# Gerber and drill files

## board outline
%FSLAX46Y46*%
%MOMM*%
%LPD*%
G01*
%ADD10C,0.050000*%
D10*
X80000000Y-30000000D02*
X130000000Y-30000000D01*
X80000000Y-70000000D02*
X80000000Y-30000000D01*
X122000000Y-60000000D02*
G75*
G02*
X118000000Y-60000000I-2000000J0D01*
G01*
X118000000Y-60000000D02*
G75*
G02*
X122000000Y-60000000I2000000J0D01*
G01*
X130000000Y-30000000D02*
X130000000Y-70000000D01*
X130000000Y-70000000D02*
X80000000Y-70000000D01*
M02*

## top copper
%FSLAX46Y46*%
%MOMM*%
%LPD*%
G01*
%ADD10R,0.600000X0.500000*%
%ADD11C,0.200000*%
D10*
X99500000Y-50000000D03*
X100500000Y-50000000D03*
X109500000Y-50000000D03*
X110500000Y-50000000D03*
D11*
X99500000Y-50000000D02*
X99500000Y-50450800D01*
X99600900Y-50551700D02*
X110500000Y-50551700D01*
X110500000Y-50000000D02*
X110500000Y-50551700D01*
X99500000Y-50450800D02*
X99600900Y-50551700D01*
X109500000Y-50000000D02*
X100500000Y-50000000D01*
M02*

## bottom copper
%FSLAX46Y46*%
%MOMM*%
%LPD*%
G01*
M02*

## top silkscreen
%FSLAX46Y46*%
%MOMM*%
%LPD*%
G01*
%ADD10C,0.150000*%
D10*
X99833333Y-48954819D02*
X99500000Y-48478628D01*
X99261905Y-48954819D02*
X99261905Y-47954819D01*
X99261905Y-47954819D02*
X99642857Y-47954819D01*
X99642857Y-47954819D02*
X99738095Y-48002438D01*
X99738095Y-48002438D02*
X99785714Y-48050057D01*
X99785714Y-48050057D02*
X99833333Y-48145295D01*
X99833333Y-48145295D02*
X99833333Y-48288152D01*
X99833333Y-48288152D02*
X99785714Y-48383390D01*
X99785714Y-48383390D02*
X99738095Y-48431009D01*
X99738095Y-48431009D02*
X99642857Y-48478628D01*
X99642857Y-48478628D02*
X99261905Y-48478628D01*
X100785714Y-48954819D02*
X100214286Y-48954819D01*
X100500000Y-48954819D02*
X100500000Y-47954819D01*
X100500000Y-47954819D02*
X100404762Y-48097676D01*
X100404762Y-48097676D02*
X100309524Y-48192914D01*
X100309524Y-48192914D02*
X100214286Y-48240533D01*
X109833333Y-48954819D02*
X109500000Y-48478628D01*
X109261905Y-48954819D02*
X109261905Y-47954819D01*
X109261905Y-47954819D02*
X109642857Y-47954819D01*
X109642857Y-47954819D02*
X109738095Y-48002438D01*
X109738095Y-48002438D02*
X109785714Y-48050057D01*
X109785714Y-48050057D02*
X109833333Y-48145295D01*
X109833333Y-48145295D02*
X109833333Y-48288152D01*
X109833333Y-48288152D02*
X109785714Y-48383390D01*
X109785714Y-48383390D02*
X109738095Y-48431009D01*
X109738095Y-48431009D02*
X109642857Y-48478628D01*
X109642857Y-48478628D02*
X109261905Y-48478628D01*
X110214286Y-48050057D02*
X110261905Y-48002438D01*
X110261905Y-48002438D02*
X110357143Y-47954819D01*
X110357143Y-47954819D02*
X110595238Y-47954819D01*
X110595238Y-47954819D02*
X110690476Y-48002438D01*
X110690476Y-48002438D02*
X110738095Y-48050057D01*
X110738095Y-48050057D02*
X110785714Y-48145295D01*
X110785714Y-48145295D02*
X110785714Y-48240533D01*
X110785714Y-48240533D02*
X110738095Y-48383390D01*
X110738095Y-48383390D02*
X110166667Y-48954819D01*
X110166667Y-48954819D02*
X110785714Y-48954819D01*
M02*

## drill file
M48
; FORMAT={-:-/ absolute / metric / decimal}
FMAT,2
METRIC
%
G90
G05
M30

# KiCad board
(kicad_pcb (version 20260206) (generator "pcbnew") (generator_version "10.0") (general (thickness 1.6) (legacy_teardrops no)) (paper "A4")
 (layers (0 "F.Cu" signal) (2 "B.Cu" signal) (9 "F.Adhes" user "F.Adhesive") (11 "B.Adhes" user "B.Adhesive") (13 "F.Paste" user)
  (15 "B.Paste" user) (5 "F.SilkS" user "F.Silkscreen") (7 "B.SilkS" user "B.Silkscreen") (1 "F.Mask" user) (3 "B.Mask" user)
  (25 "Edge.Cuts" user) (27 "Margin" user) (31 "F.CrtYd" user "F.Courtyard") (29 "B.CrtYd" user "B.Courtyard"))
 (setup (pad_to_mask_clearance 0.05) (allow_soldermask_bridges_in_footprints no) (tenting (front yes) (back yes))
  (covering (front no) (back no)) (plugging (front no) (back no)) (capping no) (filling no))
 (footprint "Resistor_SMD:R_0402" (layer "F.Cu") (at 100 50)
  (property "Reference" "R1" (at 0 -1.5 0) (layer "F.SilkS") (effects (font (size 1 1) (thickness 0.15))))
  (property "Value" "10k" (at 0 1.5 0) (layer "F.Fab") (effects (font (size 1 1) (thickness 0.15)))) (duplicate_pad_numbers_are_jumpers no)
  (pad "1" smd rect (at -0.5 0) (size 0.6 0.5) (layers "F.Cu" "F.Mask" "F.Paste") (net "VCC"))
  (pad "2" smd rect (at 0.5 0) (size 0.6 0.5) (layers "F.Cu" "F.Mask" "F.Paste") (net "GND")))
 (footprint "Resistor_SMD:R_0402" (layer "F.Cu") (at 110 50)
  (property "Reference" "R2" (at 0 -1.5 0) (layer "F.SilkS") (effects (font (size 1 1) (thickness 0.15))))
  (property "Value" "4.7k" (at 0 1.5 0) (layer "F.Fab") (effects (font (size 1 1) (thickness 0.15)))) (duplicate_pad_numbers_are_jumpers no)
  (pad "1" smd rect (at -0.5 0) (size 0.6 0.5) (layers "F.Cu" "F.Mask" "F.Paste") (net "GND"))
  (pad "2" smd rect (at 0.5 0) (size 0.6 0.5) (layers "F.Cu" "F.Mask" "F.Paste") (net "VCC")))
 (gr_line (start 80 30) (end 130 30) (stroke (width 0.05) (type default)) (layer "Edge.Cuts"))
 (gr_line (start 80 70) (end 80 30) (stroke (width 0.05) (type default)) (layer "Edge.Cuts"))
 (gr_circle (center 120 60) (end 122 60) (stroke (width 0.05) (type default)) (fill no) (layer "Edge.Cuts"))
 (gr_line (start 130 30) (end 130 70) (stroke (width 0.05) (type default)) (layer "Edge.Cuts"))
 (gr_line (start 130 70) (end 80 70) (stroke (width 0.05) (type default)) (layer "Edge.Cuts"))
 (segment (start 99.5 50) (end 99.5 50.4508) (width 0.2) (layer "F.Cu") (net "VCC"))
 (segment (start 99.6009 50.5517) (end 110.5 50.5517) (width 0.2) (layer "F.Cu") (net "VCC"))
 (segment (start 110.5 50) (end 110.5 50.5517) (width 0.2) (layer "F.Cu") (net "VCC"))
 (segment (start 99.5 50.4508) (end 99.6009 50.5517) (width 0.2) (layer "F.Cu") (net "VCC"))
 (segment (start 109.5 50) (end 100.5 50) (width 0.2) (layer "F.Cu") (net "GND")))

